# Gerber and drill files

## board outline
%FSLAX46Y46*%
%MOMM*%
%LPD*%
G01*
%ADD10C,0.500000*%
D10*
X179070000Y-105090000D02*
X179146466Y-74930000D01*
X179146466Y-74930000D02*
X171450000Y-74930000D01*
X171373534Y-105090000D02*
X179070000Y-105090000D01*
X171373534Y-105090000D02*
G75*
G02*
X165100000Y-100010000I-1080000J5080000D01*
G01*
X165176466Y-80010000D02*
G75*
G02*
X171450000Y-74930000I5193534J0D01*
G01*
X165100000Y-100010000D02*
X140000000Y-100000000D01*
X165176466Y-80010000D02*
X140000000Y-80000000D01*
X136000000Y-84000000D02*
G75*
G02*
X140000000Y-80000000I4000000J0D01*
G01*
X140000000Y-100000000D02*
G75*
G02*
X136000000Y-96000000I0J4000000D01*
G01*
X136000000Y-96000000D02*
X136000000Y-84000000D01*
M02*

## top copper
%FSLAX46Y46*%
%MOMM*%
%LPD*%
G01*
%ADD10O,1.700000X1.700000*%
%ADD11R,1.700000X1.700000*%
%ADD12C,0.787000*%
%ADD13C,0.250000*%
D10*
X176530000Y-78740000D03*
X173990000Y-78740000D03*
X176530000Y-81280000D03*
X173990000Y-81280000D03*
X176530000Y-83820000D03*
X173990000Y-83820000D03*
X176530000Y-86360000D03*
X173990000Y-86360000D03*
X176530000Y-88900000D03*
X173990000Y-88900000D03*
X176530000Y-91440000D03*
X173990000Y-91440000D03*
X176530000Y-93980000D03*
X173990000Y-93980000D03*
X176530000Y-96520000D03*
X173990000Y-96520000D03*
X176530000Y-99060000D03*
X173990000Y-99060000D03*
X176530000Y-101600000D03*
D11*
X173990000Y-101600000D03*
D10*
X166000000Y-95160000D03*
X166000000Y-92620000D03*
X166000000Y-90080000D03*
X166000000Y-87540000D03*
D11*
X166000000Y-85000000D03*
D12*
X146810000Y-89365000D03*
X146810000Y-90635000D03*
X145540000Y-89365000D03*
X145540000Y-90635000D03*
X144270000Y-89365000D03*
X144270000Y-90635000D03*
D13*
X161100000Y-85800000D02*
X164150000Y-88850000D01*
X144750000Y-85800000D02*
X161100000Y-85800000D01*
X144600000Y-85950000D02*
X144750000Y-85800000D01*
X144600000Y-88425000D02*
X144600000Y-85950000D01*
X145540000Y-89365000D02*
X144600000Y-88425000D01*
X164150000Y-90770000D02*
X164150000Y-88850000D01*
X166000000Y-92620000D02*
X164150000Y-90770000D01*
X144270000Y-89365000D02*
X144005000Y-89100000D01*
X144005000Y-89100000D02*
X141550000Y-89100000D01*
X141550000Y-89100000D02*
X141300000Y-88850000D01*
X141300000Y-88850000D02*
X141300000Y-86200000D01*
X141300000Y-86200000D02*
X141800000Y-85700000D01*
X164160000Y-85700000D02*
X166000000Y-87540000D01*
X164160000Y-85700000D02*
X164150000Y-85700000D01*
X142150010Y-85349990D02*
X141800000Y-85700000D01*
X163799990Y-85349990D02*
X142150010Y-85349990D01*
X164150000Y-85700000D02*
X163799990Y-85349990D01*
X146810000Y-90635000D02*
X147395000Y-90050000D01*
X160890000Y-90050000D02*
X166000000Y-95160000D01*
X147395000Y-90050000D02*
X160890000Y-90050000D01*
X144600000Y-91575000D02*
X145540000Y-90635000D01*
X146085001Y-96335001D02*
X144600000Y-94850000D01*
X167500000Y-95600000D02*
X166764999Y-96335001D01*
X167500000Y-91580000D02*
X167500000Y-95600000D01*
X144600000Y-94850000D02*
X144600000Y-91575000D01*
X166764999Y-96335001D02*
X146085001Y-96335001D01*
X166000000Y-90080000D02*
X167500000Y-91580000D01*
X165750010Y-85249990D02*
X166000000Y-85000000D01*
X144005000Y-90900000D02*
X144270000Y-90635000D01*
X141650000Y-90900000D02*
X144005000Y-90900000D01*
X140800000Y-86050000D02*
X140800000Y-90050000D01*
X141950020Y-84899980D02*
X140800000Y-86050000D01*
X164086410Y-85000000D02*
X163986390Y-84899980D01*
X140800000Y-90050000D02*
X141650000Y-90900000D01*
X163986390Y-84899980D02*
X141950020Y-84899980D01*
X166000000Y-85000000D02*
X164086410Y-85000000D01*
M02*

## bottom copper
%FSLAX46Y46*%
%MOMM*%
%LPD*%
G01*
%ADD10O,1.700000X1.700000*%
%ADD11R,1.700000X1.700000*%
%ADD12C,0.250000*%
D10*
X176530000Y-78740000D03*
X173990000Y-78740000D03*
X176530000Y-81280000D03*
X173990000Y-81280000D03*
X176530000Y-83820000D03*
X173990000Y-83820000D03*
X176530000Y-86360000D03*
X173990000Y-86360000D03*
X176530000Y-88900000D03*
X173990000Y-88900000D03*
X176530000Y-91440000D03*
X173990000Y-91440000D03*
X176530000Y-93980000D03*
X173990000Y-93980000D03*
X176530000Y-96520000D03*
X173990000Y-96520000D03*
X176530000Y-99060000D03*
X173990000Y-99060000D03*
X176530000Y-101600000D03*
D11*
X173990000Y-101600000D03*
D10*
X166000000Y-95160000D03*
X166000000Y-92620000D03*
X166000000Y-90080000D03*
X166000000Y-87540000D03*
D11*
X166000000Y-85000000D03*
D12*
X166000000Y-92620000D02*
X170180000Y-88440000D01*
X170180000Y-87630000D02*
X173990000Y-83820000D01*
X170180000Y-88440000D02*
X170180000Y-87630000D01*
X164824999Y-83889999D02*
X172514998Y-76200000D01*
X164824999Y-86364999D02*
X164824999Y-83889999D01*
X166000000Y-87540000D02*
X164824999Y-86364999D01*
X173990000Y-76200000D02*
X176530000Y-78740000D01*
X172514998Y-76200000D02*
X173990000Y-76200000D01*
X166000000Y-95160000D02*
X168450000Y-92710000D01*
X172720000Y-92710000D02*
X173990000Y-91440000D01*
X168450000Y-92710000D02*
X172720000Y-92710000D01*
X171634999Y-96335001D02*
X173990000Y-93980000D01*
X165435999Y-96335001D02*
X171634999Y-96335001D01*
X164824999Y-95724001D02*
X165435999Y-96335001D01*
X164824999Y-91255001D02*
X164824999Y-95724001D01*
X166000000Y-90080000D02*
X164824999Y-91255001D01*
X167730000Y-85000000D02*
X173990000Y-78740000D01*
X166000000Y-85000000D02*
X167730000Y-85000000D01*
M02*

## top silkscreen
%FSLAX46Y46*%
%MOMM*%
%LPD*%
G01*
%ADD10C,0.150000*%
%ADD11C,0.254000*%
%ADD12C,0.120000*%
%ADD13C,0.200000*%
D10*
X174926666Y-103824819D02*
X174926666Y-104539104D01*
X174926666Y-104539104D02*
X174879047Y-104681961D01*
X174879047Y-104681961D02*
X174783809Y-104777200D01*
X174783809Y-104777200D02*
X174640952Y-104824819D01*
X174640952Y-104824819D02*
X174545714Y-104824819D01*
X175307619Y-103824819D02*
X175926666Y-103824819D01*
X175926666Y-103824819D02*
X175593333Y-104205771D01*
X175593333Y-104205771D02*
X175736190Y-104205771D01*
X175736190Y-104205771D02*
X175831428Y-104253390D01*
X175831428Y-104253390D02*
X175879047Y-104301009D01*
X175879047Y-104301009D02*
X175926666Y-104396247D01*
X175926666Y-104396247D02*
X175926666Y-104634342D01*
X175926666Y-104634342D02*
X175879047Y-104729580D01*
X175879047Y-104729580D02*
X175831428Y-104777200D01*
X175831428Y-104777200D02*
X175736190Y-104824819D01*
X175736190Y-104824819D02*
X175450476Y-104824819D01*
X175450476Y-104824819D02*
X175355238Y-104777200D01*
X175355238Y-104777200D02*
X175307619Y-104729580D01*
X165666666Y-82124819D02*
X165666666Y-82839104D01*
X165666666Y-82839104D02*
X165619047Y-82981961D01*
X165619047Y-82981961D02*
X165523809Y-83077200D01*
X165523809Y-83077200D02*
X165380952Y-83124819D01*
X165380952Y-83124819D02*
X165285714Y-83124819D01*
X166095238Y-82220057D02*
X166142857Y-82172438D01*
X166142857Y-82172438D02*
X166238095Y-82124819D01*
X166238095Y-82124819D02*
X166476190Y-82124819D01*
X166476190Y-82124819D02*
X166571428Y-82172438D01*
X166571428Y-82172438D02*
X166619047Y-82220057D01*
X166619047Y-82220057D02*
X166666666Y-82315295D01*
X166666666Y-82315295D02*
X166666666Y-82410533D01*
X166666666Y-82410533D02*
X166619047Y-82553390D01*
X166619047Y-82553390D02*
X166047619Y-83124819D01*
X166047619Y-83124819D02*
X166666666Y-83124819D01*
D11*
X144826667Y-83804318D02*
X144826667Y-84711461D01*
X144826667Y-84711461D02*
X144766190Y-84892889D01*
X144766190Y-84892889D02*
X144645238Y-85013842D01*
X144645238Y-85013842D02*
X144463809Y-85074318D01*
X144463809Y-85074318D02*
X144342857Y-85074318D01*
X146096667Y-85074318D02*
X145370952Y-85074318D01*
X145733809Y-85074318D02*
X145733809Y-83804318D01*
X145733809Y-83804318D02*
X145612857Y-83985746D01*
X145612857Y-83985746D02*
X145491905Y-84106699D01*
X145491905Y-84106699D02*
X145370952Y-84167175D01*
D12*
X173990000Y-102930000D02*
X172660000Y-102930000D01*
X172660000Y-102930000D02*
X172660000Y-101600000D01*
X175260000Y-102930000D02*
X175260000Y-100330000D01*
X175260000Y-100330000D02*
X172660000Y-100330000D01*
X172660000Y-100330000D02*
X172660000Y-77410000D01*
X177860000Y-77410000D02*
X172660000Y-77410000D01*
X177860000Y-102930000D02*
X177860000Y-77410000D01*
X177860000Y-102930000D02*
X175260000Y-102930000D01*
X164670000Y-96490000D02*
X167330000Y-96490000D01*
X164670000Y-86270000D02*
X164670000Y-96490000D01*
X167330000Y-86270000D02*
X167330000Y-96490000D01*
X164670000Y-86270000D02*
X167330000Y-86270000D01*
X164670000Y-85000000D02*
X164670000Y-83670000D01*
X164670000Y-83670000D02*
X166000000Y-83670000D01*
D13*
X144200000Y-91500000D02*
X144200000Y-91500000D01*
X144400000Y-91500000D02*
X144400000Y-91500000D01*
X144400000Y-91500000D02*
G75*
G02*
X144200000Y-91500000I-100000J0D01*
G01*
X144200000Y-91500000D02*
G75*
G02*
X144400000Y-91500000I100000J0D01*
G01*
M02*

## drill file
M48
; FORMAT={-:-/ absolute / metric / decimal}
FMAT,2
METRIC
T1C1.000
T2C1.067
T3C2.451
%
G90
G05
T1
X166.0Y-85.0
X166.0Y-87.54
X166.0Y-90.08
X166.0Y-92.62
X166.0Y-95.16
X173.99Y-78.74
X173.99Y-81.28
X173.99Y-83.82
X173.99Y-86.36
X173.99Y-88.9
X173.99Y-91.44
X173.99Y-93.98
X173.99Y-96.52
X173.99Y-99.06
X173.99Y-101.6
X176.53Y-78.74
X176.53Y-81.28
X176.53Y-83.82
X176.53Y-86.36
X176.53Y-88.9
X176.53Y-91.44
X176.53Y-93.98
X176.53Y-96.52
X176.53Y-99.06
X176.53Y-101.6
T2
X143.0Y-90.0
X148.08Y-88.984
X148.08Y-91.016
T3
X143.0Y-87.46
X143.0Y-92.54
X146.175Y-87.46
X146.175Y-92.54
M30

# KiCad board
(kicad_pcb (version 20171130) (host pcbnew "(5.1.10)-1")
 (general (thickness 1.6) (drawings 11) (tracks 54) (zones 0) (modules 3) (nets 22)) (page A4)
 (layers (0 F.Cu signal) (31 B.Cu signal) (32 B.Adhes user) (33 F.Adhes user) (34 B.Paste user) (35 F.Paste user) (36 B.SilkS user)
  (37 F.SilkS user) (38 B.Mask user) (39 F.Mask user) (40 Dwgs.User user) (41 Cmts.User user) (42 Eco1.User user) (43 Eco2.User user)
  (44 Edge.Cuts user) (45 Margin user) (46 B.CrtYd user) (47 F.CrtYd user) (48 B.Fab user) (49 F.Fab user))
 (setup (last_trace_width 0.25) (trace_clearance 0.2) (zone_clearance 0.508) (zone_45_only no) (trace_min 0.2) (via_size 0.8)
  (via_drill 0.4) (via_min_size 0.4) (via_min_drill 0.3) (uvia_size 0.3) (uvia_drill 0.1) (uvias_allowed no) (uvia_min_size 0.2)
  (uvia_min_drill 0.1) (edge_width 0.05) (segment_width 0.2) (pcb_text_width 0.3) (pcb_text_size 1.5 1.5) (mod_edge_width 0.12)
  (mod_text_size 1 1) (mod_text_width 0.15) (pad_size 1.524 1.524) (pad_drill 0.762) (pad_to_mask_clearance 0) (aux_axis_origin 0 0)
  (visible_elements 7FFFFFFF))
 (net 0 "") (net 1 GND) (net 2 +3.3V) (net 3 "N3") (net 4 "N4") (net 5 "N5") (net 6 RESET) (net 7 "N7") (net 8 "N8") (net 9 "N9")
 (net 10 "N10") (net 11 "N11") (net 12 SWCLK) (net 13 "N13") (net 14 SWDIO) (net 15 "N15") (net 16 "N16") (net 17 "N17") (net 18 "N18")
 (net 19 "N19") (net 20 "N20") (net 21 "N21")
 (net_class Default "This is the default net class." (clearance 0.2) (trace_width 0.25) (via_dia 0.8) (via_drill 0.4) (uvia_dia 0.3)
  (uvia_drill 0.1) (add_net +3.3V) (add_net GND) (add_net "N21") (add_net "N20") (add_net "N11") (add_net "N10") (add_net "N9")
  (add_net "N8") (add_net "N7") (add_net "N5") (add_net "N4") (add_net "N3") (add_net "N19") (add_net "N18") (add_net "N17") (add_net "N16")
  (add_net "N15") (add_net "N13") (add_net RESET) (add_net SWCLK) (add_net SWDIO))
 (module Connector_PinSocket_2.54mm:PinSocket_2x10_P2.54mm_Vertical (layer F.Cu) (at 173.99 101.6 180)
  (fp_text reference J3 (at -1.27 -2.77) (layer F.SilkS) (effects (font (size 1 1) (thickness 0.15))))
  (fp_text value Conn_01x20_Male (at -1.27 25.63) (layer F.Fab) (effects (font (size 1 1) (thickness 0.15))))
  (fp_line (start 0 -1.33) (end 1.33 -1.33) (layer F.SilkS) (width 0.12))
  (fp_line (start 1.33 -1.33) (end 1.33 0) (layer F.SilkS) (width 0.12))
  (fp_line (start -1.27 -1.33) (end -1.27 1.27) (layer F.SilkS) (width 0.12))
  (fp_line (start -1.27 1.27) (end 1.33 1.27) (layer F.SilkS) (width 0.12))
  (fp_line (start 1.33 1.27) (end 1.33 24.19) (layer F.SilkS) (width 0.12))
  (fp_line (start -3.87 24.19) (end 1.33 24.19) (layer F.SilkS) (width 0.12))
  (fp_line (start -3.87 -1.33) (end -3.87 24.19) (layer F.SilkS) (width 0.12))
  (fp_line (start -3.87 -1.33) (end -1.27 -1.33) (layer F.SilkS) (width 0.12))
  (pad 20 thru_hole oval (at -2.54 22.86 180) (size 1.7 1.7) (drill 1) (layers *.Cu *.Mask) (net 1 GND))
  (pad 19 thru_hole oval (at 0 22.86 180) (size 1.7 1.7) (drill 1) (layers *.Cu *.Mask) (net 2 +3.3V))
  (pad 18 thru_hole oval (at -2.54 20.32 180) (size 1.7 1.7) (drill 1) (layers *.Cu *.Mask) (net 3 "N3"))
  (pad 17 thru_hole oval (at 0 20.32 180) (size 1.7 1.7) (drill 1) (layers *.Cu *.Mask) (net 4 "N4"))
  (pad 16 thru_hole oval (at -2.54 17.78 180) (size 1.7 1.7) (drill 1) (layers *.Cu *.Mask) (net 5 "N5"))
  (pad 15 thru_hole oval (at 0 17.78 180) (size 1.7 1.7) (drill 1) (layers *.Cu *.Mask) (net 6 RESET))
  (pad 14 thru_hole oval (at -2.54 15.24 180) (size 1.7 1.7) (drill 1) (layers *.Cu *.Mask) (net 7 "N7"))
  (pad 13 thru_hole oval (at 0 15.24 180) (size 1.7 1.7) (drill 1) (layers *.Cu *.Mask) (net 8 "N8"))
  (pad 12 thru_hole oval (at -2.54 12.7 180) (size 1.7 1.7) (drill 1) (layers *.Cu *.Mask) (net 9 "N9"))
  (pad 11 thru_hole oval (at 0 12.7 180) (size 1.7 1.7) (drill 1) (layers *.Cu *.Mask) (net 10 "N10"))
  (pad 10 thru_hole oval (at -2.54 10.16 180) (size 1.7 1.7) (drill 1) (layers *.Cu *.Mask) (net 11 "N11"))
  (pad 9 thru_hole oval (at 0 10.16 180) (size 1.7 1.7) (drill 1) (layers *.Cu *.Mask) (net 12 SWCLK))
  (pad 8 thru_hole oval (at -2.54 7.62 180) (size 1.7 1.7) (drill 1) (layers *.Cu *.Mask) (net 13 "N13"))
  (pad 7 thru_hole oval (at 0 7.62 180) (size 1.7 1.7) (drill 1) (layers *.Cu *.Mask) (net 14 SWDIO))
  (pad 6 thru_hole oval (at -2.54 5.08 180) (size 1.7 1.7) (drill 1) (layers *.Cu *.Mask) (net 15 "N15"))
  (pad 5 thru_hole oval (at 0 5.08 180) (size 1.7 1.7) (drill 1) (layers *.Cu *.Mask) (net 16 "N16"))
  (pad 4 thru_hole oval (at -2.54 2.54 180) (size 1.7 1.7) (drill 1) (layers *.Cu *.Mask) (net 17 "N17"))
  (pad 3 thru_hole oval (at 0 2.54 180) (size 1.7 1.7) (drill 1) (layers *.Cu *.Mask) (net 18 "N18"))
  (pad 2 thru_hole oval (at -2.54 0 180) (size 1.7 1.7) (drill 1) (layers *.Cu *.Mask) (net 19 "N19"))
  (pad 1 thru_hole rect (at 0 0 180) (size 1.7 1.7) (drill 1) (layers *.Cu *.Mask) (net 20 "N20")))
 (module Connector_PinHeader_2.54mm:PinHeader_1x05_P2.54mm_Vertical (layer F.Cu) (at 166 85)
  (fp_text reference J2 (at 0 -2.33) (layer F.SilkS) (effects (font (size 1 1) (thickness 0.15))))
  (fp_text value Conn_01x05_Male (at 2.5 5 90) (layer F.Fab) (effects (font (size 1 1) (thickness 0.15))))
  (fp_line (start -1.33 11.49) (end 1.33 11.49) (layer F.SilkS) (width 0.12))
  (fp_line (start -1.33 1.27) (end -1.33 11.49) (layer F.SilkS) (width 0.12))
  (fp_line (start 1.33 1.27) (end 1.33 11.49) (layer F.SilkS) (width 0.12))
  (fp_line (start -1.33 1.27) (end 1.33 1.27) (layer F.SilkS) (width 0.12))
  (fp_line (start -1.33 0) (end -1.33 -1.33) (layer F.SilkS) (width 0.12))
  (fp_line (start -1.33 -1.33) (end 0 -1.33) (layer F.SilkS) (width 0.12))
  (pad 5 thru_hole oval (at 0 10.16) (size 1.7 1.7) (drill 1) (layers *.Cu *.Mask) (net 12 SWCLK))
  (pad 4 thru_hole oval (at 0 7.62) (size 1.7 1.7) (drill 1) (layers *.Cu *.Mask) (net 6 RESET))
  (pad 3 thru_hole oval (at 0 5.08) (size 1.7 1.7) (drill 1) (layers *.Cu *.Mask) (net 14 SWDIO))
  (pad 2 thru_hole oval (at 0 2.54) (size 1.7 1.7) (drill 1) (layers *.Cu *.Mask) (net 1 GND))
  (pad 1 thru_hole rect (at 0 0) (size 1.7 1.7) (drill 1) (layers *.Cu *.Mask) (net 2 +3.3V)))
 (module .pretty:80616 (layer F.Cu) (at 143 90)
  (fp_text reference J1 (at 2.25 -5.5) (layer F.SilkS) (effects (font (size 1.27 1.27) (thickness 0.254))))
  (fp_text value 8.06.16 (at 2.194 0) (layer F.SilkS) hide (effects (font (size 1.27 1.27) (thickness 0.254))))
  (fp_line (start 1.2 1.5) (end 1.2 1.5) (layer F.SilkS) (width 0.2))
  (fp_line (start 1.4 1.5) (end 1.4 1.5) (layer F.SilkS) (width 0.2))
  (fp_arc (start 1.3 1.5) (end 1.4 1.5) (angle 180) (layer F.SilkS) (width 0.2))
  (fp_arc (start 1.3 1.5) (end 1.2 1.5) (angle 180) (layer F.SilkS) (width 0.2))
  (pad 13 np_thru_hole circle (at 5.08 1.016) (size 1.067 0) (drill 1.067) (layers *.Cu *.Mask))
  (pad 12 np_thru_hole circle (at 5.08 -1.016) (size 1.067 0) (drill 1.067) (layers *.Cu *.Mask))
  (pad 11 np_thru_hole circle (at 0 0) (size 1.067 0) (drill 1.067) (layers *.Cu *.Mask))
  (pad 10 np_thru_hole circle (at 3.175 2.54) (size 2.451 0) (drill 2.451) (layers *.Cu *.Mask))
  (pad 9 np_thru_hole circle (at 0 2.54) (size 2.451 0) (drill 2.451) (layers *.Cu *.Mask))
  (pad 8 np_thru_hole circle (at 3.175 -2.54) (size 2.451 0) (drill 2.451) (layers *.Cu *.Mask))
  (pad 7 np_thru_hole circle (at 0 -2.54) (size 2.451 0) (drill 2.451) (layers *.Cu *.Mask))
  (pad 6 smd circle (at 3.81 -0.635 90) (size 0.787 0.787) (layers F.Cu F.Paste F.Mask) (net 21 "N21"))
  (pad 5 smd circle (at 3.81 0.635 90) (size 0.787 0.787) (layers F.Cu F.Paste F.Mask) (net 12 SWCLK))
  (pad 4 smd circle (at 2.54 -0.635 90) (size 0.787 0.787) (layers F.Cu F.Paste F.Mask) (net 6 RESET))
  (pad 3 smd circle (at 2.54 0.635 90) (size 0.787 0.787) (layers F.Cu F.Paste F.Mask) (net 14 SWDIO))
  (pad 2 smd circle (at 1.27 -0.635 90) (size 0.787 0.787) (layers F.Cu F.Paste F.Mask) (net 1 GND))
  (pad 1 smd circle (at 1.27 0.635 90) (size 0.787 0.787) (layers F.Cu F.Paste F.Mask) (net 2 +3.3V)))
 (gr_line (start 179.07 105.09) (end 179.146466 74.93) (layer Edge.Cuts) (width 0.5))
 (gr_line (start 179.146466 74.93) (end 171.45 74.93) (layer Edge.Cuts) (width 0.5))
 (gr_line (start 171.373534 105.09) (end 179.07 105.09) (layer Edge.Cuts) (width 0.5))
 (gr_arc (start 170.293534 100.01) (end 171.373534 105.09) (angle 102.0022949) (layer Edge.Cuts) (width 0.5))
 (gr_arc (start 170.37 80.01) (end 171.45 74.93) (angle -102.0022949) (layer Edge.Cuts) (width 0.5))
 (gr_line (start 165.1 100.01) (end 140 100) (layer Edge.Cuts) (width 0.5))
 (gr_line (start 165.176466 80.01) (end 140 80) (layer Edge.Cuts) (width 0.5))
 (gr_arc (start 140 84) (end 140 80) (angle -90) (layer Edge.Cuts) (width 0.5))
 (gr_arc (start 140 96) (end 136 96) (angle -90) (layer Edge.Cuts) (width 0.5))
 (gr_line (start 136 96) (end 136 84) (layer Edge.Cuts) (width 0.5))
 (segment (start 161.1 85.8) (end 164.15 88.85) (width 0.25) (layer F.Cu) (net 6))
 (segment (start 144.75 85.8) (end 161.1 85.8) (width 0.25) (layer F.Cu) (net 6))
 (segment (start 144.6 85.95) (end 144.75 85.8) (width 0.25) (layer F.Cu) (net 6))
 (segment (start 144.6 88.425) (end 144.6 85.95) (width 0.25) (layer F.Cu) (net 6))
 (segment (start 145.54 89.365) (end 144.6 88.425) (width 0.25) (layer F.Cu) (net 6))
 (segment (start 164.15 90.77) (end 164.15 88.85) (width 0.25) (layer F.Cu) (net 6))
 (segment (start 166 92.62) (end 164.15 90.77) (width 0.25) (layer F.Cu) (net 6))
 (segment (start 166 92.62) (end 170.18 88.44) (width 0.25) (layer B.Cu) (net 6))
 (segment (start 170.18 87.63) (end 173.99 83.82) (width 0.25) (layer B.Cu) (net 6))
 (segment (start 170.18 88.44) (end 170.18 87.63) (width 0.25) (layer B.Cu) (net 6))
 (segment (start 144.27 89.365) (end 144.005 89.1) (width 0.25) (layer F.Cu) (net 1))
 (segment (start 144.005 89.1) (end 141.55 89.1) (width 0.25) (layer F.Cu) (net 1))
 (segment (start 141.55 89.1) (end 141.3 88.85) (width 0.25) (layer F.Cu) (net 1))
 (segment (start 141.3 88.85) (end 141.3 86.2) (width 0.25) (layer F.Cu) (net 1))
 (segment (start 141.3 86.2) (end 141.8 85.7) (width 0.25) (layer F.Cu) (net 1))
 (segment (start 164.16 85.7) (end 166 87.54) (width 0.25) (layer F.Cu) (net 1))
 (segment (start 164.16 85.7) (end 164.15 85.7) (width 0.25) (layer F.Cu) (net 1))
 (segment (start 142.15001 85.34999) (end 141.8 85.7) (width 0.25) (layer F.Cu) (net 1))
 (segment (start 163.79999 85.34999) (end 142.15001 85.34999) (width 0.25) (layer F.Cu) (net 1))
 (segment (start 164.15 85.7) (end 163.79999 85.34999) (width 0.25) (layer F.Cu) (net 1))
 (segment (start 164.824999 83.889999) (end 172.514998 76.2) (width 0.25) (layer B.Cu) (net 1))
 (segment (start 164.824999 86.364999) (end 164.824999 83.889999) (width 0.25) (layer B.Cu) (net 1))
 (segment (start 166 87.54) (end 164.824999 86.364999) (width 0.25) (layer B.Cu) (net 1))
 (segment (start 173.99 76.2) (end 176.53 78.74) (width 0.25) (layer B.Cu) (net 1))
 (segment (start 172.514998 76.2) (end 173.99 76.2) (width 0.25) (layer B.Cu) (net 1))
 (segment (start 146.81 90.635) (end 147.395 90.05) (width 0.25) (layer F.Cu) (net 12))
 (segment (start 160.89 90.05) (end 166 95.16) (width 0.25) (layer F.Cu) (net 12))
 (segment (start 147.395 90.05) (end 160.89 90.05) (width 0.25) (layer F.Cu) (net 12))
 (segment (start 166 95.16) (end 168.45 92.71) (width 0.25) (layer B.Cu) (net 12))
 (segment (start 172.72 92.71) (end 173.99 91.44) (width 0.25) (layer B.Cu) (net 12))
 (segment (start 168.45 92.71) (end 172.72 92.71) (width 0.25) (layer B.Cu) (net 12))
 (segment (start 144.6 91.575) (end 145.54 90.635) (width 0.25) (layer F.Cu) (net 14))
 (segment (start 146.085001 96.335001) (end 144.6 94.85) (width 0.25) (layer F.Cu) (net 14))
 (segment (start 167.5 95.6) (end 166.764999 96.335001) (width 0.25) (layer F.Cu) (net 14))
 (segment (start 167.5 91.58) (end 167.5 95.6) (width 0.25) (layer F.Cu) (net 14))
 (segment (start 144.6 94.85) (end 144.6 91.575) (width 0.25) (layer F.Cu) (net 14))
 (segment (start 166.764999 96.335001) (end 146.085001 96.335001) (width 0.25) (layer F.Cu) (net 14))
 (segment (start 166 90.08) (end 167.5 91.58) (width 0.25) (layer F.Cu) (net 14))
 (segment (start 171.634999 96.335001) (end 173.99 93.98) (width 0.25) (layer B.Cu) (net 14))
 (segment (start 165.435999 96.335001) (end 171.634999 96.335001) (width 0.25) (layer B.Cu) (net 14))
 (segment (start 164.824999 95.724001) (end 165.435999 96.335001) (width 0.25) (layer B.Cu) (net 14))
 (segment (start 164.824999 91.255001) (end 164.824999 95.724001) (width 0.25) (layer B.Cu) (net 14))
 (segment (start 166 90.08) (end 164.824999 91.255001) (width 0.25) (layer B.Cu) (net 14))
 (segment (start 165.75001 85.24999) (end 166 85) (width 0.25) (layer F.Cu) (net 2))
 (segment (start 144.005 90.9) (end 144.27 90.635) (width 0.25) (layer F.Cu) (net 2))
 (segment (start 141.65 90.9) (end 144.005 90.9) (width 0.25) (layer F.Cu) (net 2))
 (segment (start 140.8 86.05) (end 140.8 90.05) (width 0.25) (layer F.Cu) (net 2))
 (segment (start 141.95002 84.89998) (end 140.8 86.05) (width 0.25) (layer F.Cu) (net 2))
 (segment (start 164.08641 85) (end 163.98639 84.89998) (width 0.25) (layer F.Cu) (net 2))
 (segment (start 140.8 90.05) (end 141.65 90.9) (width 0.25) (layer F.Cu) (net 2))
 (segment (start 163.98639 84.89998) (end 141.95002 84.89998) (width 0.25) (layer F.Cu) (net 2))
 (segment (start 166 85) (end 164.08641 85) (width 0.25) (layer F.Cu) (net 2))
 (segment (start 167.73 85) (end 173.99 78.74) (width 0.25) (layer B.Cu) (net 2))
 (segment (start 166 85) (end 167.73 85) (width 0.25) (layer B.Cu) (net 2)))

